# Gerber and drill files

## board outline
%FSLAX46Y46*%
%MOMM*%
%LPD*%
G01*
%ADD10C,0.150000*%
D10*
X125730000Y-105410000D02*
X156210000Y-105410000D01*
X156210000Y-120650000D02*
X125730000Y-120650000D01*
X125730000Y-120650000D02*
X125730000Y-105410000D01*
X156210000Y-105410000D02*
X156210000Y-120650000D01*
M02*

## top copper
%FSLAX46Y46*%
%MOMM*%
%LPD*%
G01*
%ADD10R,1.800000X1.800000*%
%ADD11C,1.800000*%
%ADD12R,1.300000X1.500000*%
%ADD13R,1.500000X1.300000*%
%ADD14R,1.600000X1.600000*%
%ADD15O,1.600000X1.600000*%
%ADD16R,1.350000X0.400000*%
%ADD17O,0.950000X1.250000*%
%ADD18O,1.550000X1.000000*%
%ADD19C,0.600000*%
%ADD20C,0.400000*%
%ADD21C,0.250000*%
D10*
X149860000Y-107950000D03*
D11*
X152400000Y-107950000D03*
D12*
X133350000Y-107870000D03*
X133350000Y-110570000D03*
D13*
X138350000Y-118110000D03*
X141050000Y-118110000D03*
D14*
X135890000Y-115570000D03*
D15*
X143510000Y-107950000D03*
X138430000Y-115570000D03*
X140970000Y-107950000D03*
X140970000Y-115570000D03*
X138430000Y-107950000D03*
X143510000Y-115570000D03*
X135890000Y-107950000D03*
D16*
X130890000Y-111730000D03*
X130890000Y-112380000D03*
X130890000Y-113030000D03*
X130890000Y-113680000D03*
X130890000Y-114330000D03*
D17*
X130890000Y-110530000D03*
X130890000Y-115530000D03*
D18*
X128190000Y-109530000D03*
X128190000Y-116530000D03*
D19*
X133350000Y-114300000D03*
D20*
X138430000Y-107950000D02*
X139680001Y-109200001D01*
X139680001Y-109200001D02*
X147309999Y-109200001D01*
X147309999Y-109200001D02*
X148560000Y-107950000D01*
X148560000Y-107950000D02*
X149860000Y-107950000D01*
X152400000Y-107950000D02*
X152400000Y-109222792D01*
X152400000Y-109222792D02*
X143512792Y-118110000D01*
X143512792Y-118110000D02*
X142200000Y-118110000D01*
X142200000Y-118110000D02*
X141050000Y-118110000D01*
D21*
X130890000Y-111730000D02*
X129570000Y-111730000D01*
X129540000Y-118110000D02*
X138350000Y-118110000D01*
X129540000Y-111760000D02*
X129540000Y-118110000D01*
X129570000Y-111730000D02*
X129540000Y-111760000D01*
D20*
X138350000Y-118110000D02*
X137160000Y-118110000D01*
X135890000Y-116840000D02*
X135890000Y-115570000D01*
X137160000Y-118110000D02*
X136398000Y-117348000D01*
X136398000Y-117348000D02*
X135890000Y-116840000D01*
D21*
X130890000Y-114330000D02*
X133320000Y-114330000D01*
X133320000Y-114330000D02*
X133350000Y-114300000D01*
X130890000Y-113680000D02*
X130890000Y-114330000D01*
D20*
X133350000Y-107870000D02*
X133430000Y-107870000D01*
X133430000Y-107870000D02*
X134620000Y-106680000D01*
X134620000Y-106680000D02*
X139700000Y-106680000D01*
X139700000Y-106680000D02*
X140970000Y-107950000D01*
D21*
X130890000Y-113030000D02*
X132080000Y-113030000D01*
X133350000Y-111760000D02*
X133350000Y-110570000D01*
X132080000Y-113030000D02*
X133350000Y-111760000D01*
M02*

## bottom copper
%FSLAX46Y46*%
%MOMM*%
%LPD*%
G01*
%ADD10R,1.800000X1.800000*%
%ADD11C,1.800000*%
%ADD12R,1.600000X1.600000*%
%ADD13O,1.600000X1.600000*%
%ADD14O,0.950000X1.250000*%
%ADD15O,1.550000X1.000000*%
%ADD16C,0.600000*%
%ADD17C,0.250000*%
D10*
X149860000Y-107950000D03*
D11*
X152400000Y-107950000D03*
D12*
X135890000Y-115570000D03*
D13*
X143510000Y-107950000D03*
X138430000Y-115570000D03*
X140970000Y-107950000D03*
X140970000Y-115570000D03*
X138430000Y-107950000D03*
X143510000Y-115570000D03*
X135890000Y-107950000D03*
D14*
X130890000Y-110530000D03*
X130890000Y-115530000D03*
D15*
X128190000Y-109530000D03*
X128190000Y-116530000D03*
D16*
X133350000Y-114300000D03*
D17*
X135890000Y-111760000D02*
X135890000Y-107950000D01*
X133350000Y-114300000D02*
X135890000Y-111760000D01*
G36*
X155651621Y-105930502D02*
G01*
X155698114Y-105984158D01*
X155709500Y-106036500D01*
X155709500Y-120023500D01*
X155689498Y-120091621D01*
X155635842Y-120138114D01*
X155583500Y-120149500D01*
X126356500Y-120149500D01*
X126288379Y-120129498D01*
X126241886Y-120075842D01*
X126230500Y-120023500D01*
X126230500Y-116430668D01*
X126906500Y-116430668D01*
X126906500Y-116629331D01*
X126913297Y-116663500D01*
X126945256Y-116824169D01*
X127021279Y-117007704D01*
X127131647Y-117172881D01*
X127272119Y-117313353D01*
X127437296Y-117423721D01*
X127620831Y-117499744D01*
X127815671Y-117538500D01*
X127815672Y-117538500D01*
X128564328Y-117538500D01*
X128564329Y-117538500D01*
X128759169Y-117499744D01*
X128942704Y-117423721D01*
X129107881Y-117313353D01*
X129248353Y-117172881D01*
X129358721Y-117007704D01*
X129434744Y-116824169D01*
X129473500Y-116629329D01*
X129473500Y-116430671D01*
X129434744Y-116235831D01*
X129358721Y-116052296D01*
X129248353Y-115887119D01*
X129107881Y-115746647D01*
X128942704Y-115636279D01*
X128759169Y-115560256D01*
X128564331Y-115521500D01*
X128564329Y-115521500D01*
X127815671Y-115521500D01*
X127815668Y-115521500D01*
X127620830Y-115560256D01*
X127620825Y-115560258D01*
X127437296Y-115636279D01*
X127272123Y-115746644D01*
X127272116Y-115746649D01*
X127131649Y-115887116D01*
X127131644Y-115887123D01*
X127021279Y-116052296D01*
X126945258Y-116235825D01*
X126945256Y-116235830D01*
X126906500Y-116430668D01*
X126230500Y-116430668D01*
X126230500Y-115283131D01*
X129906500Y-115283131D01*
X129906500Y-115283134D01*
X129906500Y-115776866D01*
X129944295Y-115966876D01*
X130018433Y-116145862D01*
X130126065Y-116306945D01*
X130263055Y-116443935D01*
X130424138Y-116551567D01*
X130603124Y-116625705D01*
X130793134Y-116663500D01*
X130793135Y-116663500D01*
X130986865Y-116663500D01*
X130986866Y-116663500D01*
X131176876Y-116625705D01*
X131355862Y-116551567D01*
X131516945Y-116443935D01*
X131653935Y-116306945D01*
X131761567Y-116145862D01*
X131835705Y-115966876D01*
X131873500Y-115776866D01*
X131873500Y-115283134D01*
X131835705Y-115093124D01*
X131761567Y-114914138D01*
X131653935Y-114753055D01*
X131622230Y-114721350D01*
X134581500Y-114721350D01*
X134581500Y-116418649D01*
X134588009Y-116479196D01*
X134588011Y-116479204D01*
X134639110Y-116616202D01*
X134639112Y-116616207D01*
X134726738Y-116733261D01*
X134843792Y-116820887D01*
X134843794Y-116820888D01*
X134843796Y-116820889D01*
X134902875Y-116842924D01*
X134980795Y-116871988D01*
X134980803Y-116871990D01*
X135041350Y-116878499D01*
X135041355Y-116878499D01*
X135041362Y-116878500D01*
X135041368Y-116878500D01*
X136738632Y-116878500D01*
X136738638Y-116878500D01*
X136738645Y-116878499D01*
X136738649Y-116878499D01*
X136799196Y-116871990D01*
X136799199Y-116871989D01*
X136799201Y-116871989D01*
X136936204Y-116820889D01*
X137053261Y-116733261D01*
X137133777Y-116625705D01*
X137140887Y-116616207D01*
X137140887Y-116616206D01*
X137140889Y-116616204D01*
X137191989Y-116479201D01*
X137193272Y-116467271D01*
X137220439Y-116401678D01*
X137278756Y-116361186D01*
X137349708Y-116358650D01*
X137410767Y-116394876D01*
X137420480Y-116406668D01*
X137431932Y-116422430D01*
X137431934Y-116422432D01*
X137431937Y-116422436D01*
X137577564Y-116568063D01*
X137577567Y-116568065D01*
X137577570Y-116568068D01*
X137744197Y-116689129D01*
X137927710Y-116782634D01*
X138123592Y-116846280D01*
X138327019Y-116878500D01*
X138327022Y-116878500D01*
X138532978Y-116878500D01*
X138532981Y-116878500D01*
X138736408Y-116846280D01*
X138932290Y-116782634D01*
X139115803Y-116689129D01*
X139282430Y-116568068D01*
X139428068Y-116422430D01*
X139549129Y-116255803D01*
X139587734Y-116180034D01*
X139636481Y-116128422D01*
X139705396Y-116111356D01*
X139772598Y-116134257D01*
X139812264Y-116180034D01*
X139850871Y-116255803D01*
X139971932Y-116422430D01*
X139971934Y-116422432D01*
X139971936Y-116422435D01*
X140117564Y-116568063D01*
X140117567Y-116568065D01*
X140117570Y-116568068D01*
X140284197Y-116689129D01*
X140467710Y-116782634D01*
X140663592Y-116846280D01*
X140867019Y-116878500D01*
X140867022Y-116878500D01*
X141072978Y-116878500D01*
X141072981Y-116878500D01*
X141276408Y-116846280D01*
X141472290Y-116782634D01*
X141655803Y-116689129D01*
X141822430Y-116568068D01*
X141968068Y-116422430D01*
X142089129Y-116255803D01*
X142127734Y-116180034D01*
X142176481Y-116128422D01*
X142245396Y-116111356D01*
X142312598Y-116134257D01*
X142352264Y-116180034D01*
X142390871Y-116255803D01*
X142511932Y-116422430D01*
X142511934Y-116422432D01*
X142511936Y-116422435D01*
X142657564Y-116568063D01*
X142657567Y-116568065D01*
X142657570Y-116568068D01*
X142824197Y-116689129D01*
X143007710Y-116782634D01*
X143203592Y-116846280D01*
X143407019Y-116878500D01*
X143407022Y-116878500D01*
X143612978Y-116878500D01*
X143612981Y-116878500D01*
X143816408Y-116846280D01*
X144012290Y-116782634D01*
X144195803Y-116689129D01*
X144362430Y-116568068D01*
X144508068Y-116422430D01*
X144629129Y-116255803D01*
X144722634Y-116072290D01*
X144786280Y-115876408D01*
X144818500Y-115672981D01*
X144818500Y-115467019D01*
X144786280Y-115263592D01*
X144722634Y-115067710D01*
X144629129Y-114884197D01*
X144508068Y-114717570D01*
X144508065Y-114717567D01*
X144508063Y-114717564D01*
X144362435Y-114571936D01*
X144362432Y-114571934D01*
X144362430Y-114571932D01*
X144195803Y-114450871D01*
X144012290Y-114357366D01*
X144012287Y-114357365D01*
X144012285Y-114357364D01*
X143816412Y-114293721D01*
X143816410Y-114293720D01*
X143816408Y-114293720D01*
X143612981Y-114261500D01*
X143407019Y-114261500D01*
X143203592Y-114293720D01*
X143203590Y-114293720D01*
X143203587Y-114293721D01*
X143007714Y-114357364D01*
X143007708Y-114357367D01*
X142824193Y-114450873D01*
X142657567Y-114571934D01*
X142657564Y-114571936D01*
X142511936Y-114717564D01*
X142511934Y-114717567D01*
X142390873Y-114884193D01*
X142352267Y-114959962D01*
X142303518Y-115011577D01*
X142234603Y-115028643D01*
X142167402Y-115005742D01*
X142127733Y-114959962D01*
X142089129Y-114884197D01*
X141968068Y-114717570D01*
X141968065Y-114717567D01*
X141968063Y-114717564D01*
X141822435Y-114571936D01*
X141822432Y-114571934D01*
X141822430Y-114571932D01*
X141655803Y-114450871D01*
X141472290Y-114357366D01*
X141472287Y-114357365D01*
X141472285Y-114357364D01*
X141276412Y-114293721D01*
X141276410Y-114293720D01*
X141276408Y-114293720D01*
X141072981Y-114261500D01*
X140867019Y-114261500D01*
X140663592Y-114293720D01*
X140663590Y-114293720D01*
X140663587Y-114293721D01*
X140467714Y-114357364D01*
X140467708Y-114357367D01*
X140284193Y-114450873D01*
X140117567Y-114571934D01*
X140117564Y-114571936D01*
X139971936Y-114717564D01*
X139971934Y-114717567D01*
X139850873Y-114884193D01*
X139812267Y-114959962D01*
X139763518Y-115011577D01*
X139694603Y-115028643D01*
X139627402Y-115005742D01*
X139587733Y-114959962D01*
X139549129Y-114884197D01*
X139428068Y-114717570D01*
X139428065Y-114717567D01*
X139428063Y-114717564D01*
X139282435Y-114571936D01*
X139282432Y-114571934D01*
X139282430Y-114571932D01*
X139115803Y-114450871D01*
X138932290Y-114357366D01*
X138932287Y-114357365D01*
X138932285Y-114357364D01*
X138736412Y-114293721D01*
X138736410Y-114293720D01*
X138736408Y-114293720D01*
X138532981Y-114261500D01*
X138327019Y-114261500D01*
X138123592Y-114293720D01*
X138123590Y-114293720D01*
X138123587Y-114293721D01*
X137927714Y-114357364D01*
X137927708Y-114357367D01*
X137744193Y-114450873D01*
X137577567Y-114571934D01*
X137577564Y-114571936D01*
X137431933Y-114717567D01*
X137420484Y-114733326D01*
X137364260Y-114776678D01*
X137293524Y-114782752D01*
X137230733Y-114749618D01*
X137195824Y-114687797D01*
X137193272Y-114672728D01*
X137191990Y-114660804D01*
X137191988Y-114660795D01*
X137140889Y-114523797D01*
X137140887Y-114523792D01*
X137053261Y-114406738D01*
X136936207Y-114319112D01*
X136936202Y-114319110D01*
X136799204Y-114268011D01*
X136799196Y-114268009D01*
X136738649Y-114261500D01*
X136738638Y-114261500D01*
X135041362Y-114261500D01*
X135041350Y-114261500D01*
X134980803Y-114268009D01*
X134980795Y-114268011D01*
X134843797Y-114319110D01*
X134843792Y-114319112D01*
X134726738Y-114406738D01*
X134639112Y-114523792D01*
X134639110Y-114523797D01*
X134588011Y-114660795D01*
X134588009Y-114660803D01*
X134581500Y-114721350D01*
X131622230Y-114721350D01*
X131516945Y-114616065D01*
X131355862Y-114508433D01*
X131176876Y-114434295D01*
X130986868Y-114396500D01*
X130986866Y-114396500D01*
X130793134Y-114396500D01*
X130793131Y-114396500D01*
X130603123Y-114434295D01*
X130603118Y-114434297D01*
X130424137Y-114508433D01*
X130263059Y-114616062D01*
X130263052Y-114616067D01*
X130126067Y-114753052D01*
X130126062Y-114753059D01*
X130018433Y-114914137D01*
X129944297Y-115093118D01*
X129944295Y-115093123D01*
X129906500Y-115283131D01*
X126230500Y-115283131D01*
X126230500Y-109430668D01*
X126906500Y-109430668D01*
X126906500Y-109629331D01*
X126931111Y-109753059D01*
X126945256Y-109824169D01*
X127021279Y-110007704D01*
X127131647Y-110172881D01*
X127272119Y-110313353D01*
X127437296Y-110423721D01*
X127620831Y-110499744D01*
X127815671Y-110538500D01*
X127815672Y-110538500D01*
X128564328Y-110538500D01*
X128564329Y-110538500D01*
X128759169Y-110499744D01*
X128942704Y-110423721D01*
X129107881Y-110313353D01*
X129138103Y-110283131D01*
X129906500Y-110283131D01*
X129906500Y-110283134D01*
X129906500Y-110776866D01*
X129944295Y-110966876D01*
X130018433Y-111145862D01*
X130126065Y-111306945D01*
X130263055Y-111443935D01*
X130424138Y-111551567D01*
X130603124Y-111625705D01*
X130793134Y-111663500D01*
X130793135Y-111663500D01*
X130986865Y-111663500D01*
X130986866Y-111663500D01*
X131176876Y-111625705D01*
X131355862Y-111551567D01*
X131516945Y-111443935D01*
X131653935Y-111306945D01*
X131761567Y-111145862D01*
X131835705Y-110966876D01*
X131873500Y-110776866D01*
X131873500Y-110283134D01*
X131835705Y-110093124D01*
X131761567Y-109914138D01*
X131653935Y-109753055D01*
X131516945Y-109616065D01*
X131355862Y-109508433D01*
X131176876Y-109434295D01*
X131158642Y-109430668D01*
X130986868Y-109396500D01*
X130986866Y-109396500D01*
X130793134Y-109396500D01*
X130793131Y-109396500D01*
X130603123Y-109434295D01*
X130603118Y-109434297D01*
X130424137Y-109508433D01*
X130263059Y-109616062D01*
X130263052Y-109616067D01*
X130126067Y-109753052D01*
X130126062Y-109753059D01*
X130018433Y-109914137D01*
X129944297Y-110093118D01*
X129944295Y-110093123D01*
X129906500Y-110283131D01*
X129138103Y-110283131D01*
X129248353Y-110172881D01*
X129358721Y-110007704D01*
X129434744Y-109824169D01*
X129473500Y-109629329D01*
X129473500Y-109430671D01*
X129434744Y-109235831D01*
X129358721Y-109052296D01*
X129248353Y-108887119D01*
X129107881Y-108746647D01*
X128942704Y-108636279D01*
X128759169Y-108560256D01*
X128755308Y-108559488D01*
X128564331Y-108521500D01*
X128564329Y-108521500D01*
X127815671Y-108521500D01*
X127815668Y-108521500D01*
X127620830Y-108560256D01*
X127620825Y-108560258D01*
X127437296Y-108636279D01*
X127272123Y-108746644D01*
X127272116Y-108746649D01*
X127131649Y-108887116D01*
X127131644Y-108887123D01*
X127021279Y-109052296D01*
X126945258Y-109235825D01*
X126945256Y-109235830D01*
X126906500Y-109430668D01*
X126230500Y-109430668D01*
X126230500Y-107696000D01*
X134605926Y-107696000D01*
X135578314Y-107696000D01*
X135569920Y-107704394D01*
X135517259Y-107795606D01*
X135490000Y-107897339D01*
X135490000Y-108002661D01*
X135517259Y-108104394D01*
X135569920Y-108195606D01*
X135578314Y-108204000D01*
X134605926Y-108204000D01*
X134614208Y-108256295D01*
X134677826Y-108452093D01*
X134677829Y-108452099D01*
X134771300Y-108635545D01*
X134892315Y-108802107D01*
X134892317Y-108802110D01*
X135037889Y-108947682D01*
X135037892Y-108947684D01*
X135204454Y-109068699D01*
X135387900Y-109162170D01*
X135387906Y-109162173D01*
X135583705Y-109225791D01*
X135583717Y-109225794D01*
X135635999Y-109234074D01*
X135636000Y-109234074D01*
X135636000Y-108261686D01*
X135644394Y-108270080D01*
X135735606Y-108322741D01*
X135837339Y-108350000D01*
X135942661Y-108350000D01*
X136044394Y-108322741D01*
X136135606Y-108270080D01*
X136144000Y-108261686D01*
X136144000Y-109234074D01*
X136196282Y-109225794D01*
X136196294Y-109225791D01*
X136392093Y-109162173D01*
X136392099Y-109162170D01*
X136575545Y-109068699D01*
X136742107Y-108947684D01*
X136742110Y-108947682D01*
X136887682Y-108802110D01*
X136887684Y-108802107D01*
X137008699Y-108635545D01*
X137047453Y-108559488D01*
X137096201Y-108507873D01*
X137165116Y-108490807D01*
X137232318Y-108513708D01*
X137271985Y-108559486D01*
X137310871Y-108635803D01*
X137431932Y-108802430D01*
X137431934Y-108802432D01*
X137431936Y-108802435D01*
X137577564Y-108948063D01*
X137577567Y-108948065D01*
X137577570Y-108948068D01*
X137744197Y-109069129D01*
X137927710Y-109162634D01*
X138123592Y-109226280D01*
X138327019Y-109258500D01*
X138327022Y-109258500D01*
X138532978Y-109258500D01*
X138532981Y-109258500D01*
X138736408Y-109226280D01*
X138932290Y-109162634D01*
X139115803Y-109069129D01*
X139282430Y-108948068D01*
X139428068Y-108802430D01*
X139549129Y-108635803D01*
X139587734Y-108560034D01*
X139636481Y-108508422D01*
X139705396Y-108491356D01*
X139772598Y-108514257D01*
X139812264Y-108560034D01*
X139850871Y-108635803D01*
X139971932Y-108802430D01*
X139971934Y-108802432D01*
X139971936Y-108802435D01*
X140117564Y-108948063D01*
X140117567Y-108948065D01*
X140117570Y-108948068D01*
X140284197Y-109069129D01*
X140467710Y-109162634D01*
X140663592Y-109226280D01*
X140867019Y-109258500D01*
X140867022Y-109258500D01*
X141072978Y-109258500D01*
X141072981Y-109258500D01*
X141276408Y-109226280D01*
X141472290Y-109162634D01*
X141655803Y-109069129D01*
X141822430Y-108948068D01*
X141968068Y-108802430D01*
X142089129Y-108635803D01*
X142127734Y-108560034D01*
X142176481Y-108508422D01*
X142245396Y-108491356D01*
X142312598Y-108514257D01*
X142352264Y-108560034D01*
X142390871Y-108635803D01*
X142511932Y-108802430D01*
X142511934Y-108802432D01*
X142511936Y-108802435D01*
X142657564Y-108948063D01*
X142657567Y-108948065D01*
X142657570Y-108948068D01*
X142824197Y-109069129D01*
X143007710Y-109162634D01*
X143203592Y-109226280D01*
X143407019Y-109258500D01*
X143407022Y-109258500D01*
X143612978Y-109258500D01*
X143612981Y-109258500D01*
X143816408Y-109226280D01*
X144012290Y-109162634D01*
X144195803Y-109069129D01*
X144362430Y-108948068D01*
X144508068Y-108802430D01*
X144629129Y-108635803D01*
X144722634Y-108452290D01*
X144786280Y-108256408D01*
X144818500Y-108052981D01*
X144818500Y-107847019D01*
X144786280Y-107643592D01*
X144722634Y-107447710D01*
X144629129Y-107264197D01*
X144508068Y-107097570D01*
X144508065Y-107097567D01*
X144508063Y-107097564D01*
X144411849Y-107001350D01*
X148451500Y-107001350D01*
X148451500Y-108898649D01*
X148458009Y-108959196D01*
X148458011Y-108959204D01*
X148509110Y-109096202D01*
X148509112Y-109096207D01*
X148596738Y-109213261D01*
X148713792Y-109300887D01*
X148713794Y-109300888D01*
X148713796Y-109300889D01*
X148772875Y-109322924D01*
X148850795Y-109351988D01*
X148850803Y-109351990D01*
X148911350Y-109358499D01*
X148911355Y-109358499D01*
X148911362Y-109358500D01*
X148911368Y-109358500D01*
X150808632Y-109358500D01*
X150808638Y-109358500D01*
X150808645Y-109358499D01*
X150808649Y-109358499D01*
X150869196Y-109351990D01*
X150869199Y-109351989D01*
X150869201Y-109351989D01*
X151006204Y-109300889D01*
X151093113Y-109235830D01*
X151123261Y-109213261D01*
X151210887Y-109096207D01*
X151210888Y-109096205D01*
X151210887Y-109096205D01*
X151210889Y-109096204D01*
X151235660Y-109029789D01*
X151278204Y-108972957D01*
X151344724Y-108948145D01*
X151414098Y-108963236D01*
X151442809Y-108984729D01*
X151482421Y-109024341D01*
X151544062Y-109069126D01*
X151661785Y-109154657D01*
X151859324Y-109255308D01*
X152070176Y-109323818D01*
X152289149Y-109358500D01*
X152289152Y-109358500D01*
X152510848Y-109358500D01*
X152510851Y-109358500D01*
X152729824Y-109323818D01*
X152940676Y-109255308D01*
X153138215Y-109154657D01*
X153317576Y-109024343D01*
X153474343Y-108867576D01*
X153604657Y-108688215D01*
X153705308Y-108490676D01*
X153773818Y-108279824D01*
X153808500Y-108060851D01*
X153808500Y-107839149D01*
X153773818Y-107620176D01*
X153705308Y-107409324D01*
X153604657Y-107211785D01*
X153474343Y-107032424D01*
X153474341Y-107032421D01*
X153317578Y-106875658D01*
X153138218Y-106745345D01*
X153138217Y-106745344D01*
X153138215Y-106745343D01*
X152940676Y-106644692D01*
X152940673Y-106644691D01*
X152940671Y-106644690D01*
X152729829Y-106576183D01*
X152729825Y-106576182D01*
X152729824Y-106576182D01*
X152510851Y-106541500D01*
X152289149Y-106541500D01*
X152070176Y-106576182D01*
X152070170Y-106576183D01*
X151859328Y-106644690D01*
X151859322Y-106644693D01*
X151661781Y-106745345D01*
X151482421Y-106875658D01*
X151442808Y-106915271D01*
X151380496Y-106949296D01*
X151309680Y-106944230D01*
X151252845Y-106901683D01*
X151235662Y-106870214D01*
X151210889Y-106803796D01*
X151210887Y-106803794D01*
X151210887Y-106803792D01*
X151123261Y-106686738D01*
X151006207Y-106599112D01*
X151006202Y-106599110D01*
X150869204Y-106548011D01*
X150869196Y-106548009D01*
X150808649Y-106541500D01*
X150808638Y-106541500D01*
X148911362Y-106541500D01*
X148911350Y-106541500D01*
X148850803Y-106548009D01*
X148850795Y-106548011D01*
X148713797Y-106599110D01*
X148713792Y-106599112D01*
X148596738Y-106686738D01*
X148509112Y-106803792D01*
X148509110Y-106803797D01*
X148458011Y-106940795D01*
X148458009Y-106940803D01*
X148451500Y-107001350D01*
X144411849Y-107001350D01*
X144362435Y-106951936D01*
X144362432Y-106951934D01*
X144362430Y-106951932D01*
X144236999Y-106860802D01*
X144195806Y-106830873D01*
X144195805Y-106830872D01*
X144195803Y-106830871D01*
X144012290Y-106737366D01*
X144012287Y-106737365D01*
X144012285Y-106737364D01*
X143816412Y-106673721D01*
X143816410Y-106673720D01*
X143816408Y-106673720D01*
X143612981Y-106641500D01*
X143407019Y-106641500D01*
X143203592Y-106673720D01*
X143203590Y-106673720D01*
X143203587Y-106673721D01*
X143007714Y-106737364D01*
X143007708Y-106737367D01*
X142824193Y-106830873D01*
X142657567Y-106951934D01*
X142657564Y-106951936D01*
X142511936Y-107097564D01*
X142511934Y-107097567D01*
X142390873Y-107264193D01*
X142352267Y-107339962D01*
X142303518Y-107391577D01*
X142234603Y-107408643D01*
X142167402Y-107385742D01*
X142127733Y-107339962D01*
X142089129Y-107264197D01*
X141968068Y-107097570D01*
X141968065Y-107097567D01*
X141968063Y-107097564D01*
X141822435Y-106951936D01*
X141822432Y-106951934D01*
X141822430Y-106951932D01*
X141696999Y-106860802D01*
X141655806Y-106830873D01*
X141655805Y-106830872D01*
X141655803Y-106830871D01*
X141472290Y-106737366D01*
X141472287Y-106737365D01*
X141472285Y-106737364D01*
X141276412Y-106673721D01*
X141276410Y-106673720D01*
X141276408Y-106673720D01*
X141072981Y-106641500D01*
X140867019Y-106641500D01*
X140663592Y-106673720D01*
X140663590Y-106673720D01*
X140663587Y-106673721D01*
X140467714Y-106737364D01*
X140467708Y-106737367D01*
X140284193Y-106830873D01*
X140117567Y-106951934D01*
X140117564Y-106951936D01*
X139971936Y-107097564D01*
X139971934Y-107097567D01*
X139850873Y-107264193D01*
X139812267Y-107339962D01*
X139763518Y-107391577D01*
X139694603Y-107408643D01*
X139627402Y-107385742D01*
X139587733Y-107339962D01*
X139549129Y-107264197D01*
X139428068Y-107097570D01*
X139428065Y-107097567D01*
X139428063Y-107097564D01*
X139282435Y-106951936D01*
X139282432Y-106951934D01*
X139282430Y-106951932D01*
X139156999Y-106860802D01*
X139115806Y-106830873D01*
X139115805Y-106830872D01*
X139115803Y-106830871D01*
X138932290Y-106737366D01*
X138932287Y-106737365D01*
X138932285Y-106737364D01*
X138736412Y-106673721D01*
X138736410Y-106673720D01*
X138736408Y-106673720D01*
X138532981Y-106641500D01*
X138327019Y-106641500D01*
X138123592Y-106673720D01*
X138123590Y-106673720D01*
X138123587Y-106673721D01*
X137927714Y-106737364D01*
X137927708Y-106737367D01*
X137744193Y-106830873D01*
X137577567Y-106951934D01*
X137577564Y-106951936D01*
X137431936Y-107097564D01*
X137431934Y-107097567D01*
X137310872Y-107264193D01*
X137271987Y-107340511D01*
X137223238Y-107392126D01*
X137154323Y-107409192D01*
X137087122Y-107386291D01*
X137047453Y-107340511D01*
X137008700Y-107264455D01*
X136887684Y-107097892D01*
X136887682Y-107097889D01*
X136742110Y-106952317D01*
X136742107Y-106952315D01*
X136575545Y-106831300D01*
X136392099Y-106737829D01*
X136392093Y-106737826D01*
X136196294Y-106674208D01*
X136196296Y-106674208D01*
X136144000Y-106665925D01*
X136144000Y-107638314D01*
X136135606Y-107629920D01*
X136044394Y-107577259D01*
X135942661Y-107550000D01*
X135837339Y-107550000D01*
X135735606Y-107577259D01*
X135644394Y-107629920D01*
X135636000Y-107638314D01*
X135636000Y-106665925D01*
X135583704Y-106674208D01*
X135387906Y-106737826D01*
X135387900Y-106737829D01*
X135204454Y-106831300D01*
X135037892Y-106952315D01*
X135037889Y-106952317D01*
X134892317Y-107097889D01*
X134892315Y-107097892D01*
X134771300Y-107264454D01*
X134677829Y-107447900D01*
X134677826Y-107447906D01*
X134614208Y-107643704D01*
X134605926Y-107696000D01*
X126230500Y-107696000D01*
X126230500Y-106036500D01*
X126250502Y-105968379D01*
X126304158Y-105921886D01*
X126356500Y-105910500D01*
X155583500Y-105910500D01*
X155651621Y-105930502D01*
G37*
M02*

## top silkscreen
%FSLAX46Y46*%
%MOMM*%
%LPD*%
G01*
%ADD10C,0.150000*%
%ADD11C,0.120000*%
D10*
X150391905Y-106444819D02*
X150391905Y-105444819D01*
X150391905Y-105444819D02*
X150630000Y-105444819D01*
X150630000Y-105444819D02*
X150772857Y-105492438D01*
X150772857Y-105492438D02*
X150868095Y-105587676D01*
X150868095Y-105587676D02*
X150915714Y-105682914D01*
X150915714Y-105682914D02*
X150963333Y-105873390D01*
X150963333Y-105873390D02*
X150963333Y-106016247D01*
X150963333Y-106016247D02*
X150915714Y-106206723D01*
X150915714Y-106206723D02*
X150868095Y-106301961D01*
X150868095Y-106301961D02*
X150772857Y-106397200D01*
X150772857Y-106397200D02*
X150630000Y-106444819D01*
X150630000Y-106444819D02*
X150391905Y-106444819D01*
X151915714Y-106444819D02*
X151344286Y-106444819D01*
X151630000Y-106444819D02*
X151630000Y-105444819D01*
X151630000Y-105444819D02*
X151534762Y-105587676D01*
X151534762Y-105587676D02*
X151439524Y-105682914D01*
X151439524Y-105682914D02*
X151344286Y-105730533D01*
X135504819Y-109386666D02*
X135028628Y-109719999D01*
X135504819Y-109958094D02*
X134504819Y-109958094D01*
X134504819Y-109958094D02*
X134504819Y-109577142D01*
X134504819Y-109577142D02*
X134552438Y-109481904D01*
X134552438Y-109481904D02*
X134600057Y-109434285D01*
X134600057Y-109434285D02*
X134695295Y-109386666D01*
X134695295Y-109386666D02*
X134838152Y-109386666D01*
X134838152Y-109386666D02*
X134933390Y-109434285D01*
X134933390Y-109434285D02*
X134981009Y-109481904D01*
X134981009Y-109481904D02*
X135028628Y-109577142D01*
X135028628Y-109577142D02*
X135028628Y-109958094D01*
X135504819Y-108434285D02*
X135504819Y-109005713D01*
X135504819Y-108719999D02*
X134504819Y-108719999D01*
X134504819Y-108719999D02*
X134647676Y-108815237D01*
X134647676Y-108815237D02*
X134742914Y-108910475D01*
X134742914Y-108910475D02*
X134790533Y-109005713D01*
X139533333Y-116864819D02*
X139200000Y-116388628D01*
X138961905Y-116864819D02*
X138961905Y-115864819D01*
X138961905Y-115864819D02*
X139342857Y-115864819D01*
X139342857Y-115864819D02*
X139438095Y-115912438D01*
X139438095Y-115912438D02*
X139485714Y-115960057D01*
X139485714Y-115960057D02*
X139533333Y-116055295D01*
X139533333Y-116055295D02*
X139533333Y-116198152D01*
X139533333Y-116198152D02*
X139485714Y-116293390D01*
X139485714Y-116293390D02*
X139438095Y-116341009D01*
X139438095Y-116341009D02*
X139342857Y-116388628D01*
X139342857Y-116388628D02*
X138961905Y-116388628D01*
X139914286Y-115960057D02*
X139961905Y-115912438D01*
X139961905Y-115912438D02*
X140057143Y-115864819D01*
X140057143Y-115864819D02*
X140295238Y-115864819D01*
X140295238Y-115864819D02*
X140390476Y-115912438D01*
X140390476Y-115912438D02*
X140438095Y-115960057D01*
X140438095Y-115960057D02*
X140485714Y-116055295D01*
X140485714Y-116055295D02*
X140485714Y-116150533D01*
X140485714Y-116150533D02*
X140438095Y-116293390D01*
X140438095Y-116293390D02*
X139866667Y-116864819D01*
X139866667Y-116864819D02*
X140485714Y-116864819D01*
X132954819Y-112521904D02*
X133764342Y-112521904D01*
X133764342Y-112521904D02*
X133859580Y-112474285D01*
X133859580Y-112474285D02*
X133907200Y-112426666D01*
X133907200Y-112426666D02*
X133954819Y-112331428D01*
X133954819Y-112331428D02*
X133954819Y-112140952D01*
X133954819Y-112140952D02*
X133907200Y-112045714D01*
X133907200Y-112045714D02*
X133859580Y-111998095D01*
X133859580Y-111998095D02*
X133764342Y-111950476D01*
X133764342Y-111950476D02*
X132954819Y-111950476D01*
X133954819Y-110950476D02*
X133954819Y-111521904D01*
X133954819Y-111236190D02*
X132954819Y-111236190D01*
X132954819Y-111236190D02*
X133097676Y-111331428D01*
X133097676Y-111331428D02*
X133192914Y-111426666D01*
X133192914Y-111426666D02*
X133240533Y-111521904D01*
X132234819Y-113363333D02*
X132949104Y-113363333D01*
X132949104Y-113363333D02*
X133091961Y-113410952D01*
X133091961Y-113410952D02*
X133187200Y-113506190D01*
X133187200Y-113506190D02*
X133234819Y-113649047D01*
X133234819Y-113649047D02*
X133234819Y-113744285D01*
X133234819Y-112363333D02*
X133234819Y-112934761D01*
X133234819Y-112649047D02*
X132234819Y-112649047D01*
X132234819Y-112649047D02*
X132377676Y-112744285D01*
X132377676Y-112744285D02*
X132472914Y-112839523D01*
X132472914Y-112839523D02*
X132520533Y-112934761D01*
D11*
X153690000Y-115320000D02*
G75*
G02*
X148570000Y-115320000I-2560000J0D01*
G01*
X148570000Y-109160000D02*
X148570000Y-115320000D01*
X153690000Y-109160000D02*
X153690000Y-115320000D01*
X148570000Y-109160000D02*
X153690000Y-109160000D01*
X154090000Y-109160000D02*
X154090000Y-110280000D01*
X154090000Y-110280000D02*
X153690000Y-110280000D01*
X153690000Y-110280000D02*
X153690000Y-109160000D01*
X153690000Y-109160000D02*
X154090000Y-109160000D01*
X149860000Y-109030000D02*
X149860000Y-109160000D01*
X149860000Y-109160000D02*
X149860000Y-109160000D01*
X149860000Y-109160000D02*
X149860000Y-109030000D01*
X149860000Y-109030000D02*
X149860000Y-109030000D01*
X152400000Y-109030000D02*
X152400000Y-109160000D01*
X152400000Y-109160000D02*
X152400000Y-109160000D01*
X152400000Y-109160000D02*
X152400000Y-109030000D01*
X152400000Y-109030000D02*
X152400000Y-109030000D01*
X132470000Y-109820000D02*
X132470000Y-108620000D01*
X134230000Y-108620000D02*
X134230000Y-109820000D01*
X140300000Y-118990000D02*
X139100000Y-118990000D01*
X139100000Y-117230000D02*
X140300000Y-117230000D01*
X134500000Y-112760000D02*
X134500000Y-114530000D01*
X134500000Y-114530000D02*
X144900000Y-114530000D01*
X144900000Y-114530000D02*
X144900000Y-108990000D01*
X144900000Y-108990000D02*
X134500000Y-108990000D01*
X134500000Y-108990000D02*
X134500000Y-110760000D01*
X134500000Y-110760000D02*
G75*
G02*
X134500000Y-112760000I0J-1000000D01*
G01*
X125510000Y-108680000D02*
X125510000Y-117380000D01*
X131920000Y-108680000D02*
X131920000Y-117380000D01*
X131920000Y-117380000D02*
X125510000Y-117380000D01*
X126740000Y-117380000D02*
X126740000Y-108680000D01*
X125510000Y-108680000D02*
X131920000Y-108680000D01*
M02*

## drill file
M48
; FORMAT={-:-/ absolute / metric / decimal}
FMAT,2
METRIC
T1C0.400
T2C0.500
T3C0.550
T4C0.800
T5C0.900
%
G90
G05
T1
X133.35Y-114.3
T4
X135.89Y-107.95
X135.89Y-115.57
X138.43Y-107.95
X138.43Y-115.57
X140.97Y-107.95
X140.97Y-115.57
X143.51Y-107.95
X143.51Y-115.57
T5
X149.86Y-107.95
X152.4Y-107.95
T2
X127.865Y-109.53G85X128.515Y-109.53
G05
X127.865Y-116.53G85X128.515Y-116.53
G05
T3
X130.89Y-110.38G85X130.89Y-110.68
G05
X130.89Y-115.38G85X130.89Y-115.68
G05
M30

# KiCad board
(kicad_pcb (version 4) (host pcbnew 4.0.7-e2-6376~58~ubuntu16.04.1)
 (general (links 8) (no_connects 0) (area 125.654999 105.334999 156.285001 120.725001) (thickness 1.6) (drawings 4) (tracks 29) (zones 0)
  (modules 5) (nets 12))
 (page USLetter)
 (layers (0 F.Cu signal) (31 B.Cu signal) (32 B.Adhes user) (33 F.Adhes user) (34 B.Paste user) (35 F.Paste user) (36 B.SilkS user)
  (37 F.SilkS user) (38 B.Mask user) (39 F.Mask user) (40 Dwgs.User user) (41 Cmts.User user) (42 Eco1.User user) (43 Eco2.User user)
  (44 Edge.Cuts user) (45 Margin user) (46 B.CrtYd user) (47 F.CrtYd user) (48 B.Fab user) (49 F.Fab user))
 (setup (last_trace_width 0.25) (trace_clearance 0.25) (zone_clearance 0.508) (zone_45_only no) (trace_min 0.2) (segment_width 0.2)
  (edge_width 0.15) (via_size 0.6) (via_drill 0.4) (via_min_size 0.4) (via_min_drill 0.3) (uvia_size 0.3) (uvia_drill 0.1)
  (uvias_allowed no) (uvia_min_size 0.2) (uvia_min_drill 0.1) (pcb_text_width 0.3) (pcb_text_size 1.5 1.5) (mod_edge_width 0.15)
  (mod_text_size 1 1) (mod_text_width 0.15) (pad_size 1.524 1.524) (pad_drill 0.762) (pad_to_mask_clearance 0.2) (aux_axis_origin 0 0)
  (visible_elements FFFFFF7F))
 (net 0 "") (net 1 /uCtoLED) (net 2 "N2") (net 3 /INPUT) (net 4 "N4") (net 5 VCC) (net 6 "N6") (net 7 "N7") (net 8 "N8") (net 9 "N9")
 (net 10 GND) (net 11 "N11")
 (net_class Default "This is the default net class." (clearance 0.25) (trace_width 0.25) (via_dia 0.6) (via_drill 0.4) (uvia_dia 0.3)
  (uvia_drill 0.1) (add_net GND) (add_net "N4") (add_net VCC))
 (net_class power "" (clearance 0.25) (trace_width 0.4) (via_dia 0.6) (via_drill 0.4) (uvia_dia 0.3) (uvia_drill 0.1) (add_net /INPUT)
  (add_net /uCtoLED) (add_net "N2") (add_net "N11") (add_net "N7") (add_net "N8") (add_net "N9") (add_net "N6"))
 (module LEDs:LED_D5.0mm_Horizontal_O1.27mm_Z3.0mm (layer F.Cu) (at 149.86 107.95)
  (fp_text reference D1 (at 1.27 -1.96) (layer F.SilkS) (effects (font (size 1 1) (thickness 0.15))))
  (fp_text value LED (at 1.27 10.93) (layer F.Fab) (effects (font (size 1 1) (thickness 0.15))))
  (fp_arc (start 1.27 7.37) (end -1.29 7.37) (angle -180) (layer F.SilkS) (width 0.12))
  (fp_line (start -1.29 1.21) (end -1.29 7.37) (layer F.SilkS) (width 0.12))
  (fp_line (start 3.83 1.21) (end 3.83 7.37) (layer F.SilkS) (width 0.12))
  (fp_line (start -1.29 1.21) (end 3.83 1.21) (layer F.SilkS) (width 0.12))
  (fp_line (start 4.23 1.21) (end 4.23 2.33) (layer F.SilkS) (width 0.12))
  (fp_line (start 4.23 2.33) (end 3.83 2.33) (layer F.SilkS) (width 0.12))
  (fp_line (start 3.83 2.33) (end 3.83 1.21) (layer F.SilkS) (width 0.12))
  (fp_line (start 3.83 1.21) (end 4.23 1.21) (layer F.SilkS) (width 0.12))
  (fp_line (start 0 1.08) (end 0 1.21) (layer F.SilkS) (width 0.12))
  (fp_line (start 0 1.21) (end 0 1.21) (layer F.SilkS) (width 0.12))
  (fp_line (start 0 1.21) (end 0 1.08) (layer F.SilkS) (width 0.12))
  (fp_line (start 0 1.08) (end 0 1.08) (layer F.SilkS) (width 0.12))
  (fp_line (start 2.54 1.08) (end 2.54 1.21) (layer F.SilkS) (width 0.12))
  (fp_line (start 2.54 1.21) (end 2.54 1.21) (layer F.SilkS) (width 0.12))
  (fp_line (start 2.54 1.21) (end 2.54 1.08) (layer F.SilkS) (width 0.12))
  (fp_line (start 2.54 1.08) (end 2.54 1.08) (layer F.SilkS) (width 0.12))
  (pad 1 thru_hole rect (at 0 0) (size 1.8 1.8) (drill 0.9) (layers *.Cu *.Mask) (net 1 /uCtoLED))
  (pad 2 thru_hole circle (at 2.54 0) (size 1.8 1.8) (drill 0.9) (layers *.Cu *.Mask) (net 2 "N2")))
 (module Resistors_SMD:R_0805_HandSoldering (layer F.Cu) (at 133.35 109.22 270)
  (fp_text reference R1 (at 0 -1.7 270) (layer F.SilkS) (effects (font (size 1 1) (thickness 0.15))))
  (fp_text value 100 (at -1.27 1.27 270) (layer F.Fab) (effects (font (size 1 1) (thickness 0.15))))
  (fp_line (start 0.6 0.88) (end -0.6 0.88) (layer F.SilkS) (width 0.12))
  (fp_line (start -0.6 -0.88) (end 0.6 -0.88) (layer F.SilkS) (width 0.12))
  (pad 1 smd rect (at -1.35 0 270) (size 1.5 1.3) (layers F.Cu F.Paste F.Mask) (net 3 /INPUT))
  (pad 2 smd rect (at 1.35 0 270) (size 1.5 1.3) (layers F.Cu F.Paste F.Mask) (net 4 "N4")))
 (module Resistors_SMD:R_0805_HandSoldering (layer F.Cu) (at 139.7 118.11)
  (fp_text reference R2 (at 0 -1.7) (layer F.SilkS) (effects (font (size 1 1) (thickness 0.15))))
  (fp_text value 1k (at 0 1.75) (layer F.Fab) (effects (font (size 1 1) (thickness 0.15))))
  (fp_line (start 0.6 0.88) (end -0.6 0.88) (layer F.SilkS) (width 0.12))
  (fp_line (start -0.6 -0.88) (end 0.6 -0.88) (layer F.SilkS) (width 0.12))
  (pad 1 smd rect (at -1.35 0) (size 1.5 1.3) (layers F.Cu F.Paste F.Mask) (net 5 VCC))
  (pad 2 smd rect (at 1.35 0) (size 1.5 1.3) (layers F.Cu F.Paste F.Mask) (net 2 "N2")))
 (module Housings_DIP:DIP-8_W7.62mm (layer F.Cu) (at 135.89 115.57 90)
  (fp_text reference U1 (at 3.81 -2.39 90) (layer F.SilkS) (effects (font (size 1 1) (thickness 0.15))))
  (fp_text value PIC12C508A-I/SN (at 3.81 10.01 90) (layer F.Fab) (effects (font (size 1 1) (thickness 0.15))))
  (fp_line (start 2.81 -1.39) (end 1.04 -1.39) (layer F.SilkS) (width 0.12))
  (fp_line (start 1.04 -1.39) (end 1.04 9.01) (layer F.SilkS) (width 0.12))
  (fp_line (start 1.04 9.01) (end 6.58 9.01) (layer F.SilkS) (width 0.12))
  (fp_line (start 6.58 9.01) (end 6.58 -1.39) (layer F.SilkS) (width 0.12))
  (fp_line (start 6.58 -1.39) (end 4.81 -1.39) (layer F.SilkS) (width 0.12))
  (fp_arc (start 3.81 -1.39) (end 2.81 -1.39) (angle -180) (layer F.SilkS) (width 0.12))
  (pad 1 thru_hole rect (at 0 0 90) (size 1.6 1.6) (drill 0.8) (layers *.Cu *.Mask) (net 5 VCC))
  (pad 5 thru_hole oval (at 7.62 7.62 90) (size 1.6 1.6) (drill 0.8) (layers *.Cu *.Mask) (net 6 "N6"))
  (pad 2 thru_hole oval (at 0 2.54 90) (size 1.6 1.6) (drill 0.8) (layers *.Cu *.Mask) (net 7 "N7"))
  (pad 6 thru_hole oval (at 7.62 5.08 90) (size 1.6 1.6) (drill 0.8) (layers *.Cu *.Mask) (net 3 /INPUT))
  (pad 3 thru_hole oval (at 0 5.08 90) (size 1.6 1.6) (drill 0.8) (layers *.Cu *.Mask) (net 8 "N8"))
  (pad 7 thru_hole oval (at 7.62 2.54 90) (size 1.6 1.6) (drill 0.8) (layers *.Cu *.Mask) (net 1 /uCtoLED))
  (pad 4 thru_hole oval (at 0 7.62 90) (size 1.6 1.6) (drill 0.8) (layers *.Cu *.Mask) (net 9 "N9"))
  (pad 8 thru_hole oval (at 7.62 0 90) (size 1.6 1.6) (drill 0.8) (layers *.Cu *.Mask) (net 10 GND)))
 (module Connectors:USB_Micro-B (layer F.Cu) (at 129.54 113.03 270)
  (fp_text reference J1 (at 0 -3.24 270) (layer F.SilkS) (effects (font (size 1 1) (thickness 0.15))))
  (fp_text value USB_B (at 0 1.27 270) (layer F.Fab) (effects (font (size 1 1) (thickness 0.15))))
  (fp_line (start -4.35 4.03) (end 4.35 4.03) (layer F.SilkS) (width 0.12))
  (fp_line (start -4.35 -2.38) (end 4.35 -2.38) (layer F.SilkS) (width 0.12))
  (fp_line (start 4.35 -2.38) (end 4.35 4.03) (layer F.SilkS) (width 0.12))
  (fp_line (start 4.35 2.8) (end -4.35 2.8) (layer F.SilkS) (width 0.12))
  (fp_line (start -4.35 4.03) (end -4.35 -2.38) (layer F.SilkS) (width 0.12))
  (pad 1 smd rect (at -1.3 -1.35) (size 1.35 0.4) (layers F.Cu F.Paste F.Mask) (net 5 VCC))
  (pad 2 smd rect (at -0.65 -1.35) (size 1.35 0.4) (layers F.Cu F.Paste F.Mask) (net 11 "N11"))
  (pad 3 smd rect (at 0 -1.35) (size 1.35 0.4) (layers F.Cu F.Paste F.Mask) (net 4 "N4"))
  (pad 4 smd rect (at 0.65 -1.35) (size 1.35 0.4) (layers F.Cu F.Paste F.Mask) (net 10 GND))
  (pad 5 smd rect (at 1.3 -1.35) (size 1.35 0.4) (layers F.Cu F.Paste F.Mask) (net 10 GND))
  (pad 6 thru_hole oval (at -2.5 -1.35) (size 0.95 1.25) (drill oval 0.55 0.85) (layers *.Cu *.Mask))
  (pad 6 thru_hole oval (at 2.5 -1.35) (size 0.95 1.25) (drill oval 0.55 0.85) (layers *.Cu *.Mask))
  (pad 6 thru_hole oval (at -3.5 1.35) (size 1.55 1) (drill oval 1.15 0.5) (layers *.Cu *.Mask))
  (pad 6 thru_hole oval (at 3.5 1.35) (size 1.55 1) (drill oval 1.15 0.5) (layers *.Cu *.Mask)))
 (gr_line (start 125.73 105.41) (end 156.21 105.41) (angle 90) (layer Edge.Cuts) (width 0.15))
 (gr_line (start 156.21 120.65) (end 125.73 120.65) (angle 90) (layer Edge.Cuts) (width 0.15))
 (gr_line (start 125.73 120.65) (end 125.73 105.41) (angle 90) (layer Edge.Cuts) (width 0.15))
 (gr_line (start 156.21 105.41) (end 156.21 120.65) (angle 90) (layer Edge.Cuts) (width 0.15))
 (segment (start 138.43 107.95) (end 139.680001 109.200001) (width 0.4) (layer F.Cu) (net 1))
 (segment (start 139.680001 109.200001) (end 147.309999 109.200001) (width 0.4) (layer F.Cu) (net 1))
 (segment (start 147.309999 109.200001) (end 148.56 107.95) (width 0.4) (layer F.Cu) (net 1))
 (segment (start 148.56 107.95) (end 149.86 107.95) (width 0.4) (layer F.Cu) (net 1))
 (segment (start 152.4 107.95) (end 152.4 109.222792) (width 0.4) (layer F.Cu) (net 2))
 (segment (start 152.4 109.222792) (end 143.512792 118.11) (width 0.4) (layer F.Cu) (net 2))
 (segment (start 143.512792 118.11) (end 142.2 118.11) (width 0.4) (layer F.Cu) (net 2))
 (segment (start 142.2 118.11) (end 141.05 118.11) (width 0.4) (layer F.Cu) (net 2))
 (segment (start 130.89 111.73) (end 129.57 111.73) (width 0.25) (layer F.Cu) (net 5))
 (segment (start 129.54 118.11) (end 138.35 118.11) (width 0.25) (layer F.Cu) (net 5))
 (segment (start 129.54 111.76) (end 129.54 118.11) (width 0.25) (layer F.Cu) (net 5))
 (segment (start 129.57 111.73) (end 129.54 111.76) (width 0.25) (layer F.Cu) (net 5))
 (segment (start 138.35 118.11) (end 137.16 118.11) (width 0.4) (layer F.Cu) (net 5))
 (segment (start 135.89 116.84) (end 135.89 115.57) (width 0.4) (layer F.Cu) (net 5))
 (segment (start 137.16 118.11) (end 136.398 117.348) (width 0.4) (layer F.Cu) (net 5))
 (segment (start 136.398 117.348) (end 135.89 116.84) (width 0.4) (layer F.Cu) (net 5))
 (segment (start 130.89 114.33) (end 133.32 114.33) (width 0.25) (layer F.Cu) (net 10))
 (segment (start 135.89 111.76) (end 135.89 107.95) (width 0.25) (layer B.Cu) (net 10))
 (segment (start 133.35 114.3) (end 135.89 111.76) (width 0.25) (layer B.Cu) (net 10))
 (via (at 133.35 114.3) (size 0.6) (drill 0.4) (layers F.Cu B.Cu) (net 10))
 (segment (start 133.32 114.33) (end 133.35 114.3) (width 0.25) (layer F.Cu) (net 10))
 (segment (start 130.89 113.68) (end 130.89 114.33) (width 0.25) (layer F.Cu) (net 10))
 (segment (start 133.35 107.87) (end 133.43 107.87) (width 0.4) (layer F.Cu) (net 3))
 (segment (start 133.43 107.87) (end 134.62 106.68) (width 0.4) (layer F.Cu) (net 3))
 (segment (start 134.62 106.68) (end 139.7 106.68) (width 0.4) (layer F.Cu) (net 3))
 (segment (start 139.7 106.68) (end 140.97 107.95) (width 0.4) (layer F.Cu) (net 3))
 (segment (start 130.89 113.03) (end 132.08 113.03) (width 0.25) (layer F.Cu) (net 4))
 (segment (start 133.35 111.76) (end 133.35 110.57) (width 0.25) (layer F.Cu) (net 4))
 (segment (start 132.08 113.03) (end 133.35 111.76) (width 0.25) (layer F.Cu) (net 4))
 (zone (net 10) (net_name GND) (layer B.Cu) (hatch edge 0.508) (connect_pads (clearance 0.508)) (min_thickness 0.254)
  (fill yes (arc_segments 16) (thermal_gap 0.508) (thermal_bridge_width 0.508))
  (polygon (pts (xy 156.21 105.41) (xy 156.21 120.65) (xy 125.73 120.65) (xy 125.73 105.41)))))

